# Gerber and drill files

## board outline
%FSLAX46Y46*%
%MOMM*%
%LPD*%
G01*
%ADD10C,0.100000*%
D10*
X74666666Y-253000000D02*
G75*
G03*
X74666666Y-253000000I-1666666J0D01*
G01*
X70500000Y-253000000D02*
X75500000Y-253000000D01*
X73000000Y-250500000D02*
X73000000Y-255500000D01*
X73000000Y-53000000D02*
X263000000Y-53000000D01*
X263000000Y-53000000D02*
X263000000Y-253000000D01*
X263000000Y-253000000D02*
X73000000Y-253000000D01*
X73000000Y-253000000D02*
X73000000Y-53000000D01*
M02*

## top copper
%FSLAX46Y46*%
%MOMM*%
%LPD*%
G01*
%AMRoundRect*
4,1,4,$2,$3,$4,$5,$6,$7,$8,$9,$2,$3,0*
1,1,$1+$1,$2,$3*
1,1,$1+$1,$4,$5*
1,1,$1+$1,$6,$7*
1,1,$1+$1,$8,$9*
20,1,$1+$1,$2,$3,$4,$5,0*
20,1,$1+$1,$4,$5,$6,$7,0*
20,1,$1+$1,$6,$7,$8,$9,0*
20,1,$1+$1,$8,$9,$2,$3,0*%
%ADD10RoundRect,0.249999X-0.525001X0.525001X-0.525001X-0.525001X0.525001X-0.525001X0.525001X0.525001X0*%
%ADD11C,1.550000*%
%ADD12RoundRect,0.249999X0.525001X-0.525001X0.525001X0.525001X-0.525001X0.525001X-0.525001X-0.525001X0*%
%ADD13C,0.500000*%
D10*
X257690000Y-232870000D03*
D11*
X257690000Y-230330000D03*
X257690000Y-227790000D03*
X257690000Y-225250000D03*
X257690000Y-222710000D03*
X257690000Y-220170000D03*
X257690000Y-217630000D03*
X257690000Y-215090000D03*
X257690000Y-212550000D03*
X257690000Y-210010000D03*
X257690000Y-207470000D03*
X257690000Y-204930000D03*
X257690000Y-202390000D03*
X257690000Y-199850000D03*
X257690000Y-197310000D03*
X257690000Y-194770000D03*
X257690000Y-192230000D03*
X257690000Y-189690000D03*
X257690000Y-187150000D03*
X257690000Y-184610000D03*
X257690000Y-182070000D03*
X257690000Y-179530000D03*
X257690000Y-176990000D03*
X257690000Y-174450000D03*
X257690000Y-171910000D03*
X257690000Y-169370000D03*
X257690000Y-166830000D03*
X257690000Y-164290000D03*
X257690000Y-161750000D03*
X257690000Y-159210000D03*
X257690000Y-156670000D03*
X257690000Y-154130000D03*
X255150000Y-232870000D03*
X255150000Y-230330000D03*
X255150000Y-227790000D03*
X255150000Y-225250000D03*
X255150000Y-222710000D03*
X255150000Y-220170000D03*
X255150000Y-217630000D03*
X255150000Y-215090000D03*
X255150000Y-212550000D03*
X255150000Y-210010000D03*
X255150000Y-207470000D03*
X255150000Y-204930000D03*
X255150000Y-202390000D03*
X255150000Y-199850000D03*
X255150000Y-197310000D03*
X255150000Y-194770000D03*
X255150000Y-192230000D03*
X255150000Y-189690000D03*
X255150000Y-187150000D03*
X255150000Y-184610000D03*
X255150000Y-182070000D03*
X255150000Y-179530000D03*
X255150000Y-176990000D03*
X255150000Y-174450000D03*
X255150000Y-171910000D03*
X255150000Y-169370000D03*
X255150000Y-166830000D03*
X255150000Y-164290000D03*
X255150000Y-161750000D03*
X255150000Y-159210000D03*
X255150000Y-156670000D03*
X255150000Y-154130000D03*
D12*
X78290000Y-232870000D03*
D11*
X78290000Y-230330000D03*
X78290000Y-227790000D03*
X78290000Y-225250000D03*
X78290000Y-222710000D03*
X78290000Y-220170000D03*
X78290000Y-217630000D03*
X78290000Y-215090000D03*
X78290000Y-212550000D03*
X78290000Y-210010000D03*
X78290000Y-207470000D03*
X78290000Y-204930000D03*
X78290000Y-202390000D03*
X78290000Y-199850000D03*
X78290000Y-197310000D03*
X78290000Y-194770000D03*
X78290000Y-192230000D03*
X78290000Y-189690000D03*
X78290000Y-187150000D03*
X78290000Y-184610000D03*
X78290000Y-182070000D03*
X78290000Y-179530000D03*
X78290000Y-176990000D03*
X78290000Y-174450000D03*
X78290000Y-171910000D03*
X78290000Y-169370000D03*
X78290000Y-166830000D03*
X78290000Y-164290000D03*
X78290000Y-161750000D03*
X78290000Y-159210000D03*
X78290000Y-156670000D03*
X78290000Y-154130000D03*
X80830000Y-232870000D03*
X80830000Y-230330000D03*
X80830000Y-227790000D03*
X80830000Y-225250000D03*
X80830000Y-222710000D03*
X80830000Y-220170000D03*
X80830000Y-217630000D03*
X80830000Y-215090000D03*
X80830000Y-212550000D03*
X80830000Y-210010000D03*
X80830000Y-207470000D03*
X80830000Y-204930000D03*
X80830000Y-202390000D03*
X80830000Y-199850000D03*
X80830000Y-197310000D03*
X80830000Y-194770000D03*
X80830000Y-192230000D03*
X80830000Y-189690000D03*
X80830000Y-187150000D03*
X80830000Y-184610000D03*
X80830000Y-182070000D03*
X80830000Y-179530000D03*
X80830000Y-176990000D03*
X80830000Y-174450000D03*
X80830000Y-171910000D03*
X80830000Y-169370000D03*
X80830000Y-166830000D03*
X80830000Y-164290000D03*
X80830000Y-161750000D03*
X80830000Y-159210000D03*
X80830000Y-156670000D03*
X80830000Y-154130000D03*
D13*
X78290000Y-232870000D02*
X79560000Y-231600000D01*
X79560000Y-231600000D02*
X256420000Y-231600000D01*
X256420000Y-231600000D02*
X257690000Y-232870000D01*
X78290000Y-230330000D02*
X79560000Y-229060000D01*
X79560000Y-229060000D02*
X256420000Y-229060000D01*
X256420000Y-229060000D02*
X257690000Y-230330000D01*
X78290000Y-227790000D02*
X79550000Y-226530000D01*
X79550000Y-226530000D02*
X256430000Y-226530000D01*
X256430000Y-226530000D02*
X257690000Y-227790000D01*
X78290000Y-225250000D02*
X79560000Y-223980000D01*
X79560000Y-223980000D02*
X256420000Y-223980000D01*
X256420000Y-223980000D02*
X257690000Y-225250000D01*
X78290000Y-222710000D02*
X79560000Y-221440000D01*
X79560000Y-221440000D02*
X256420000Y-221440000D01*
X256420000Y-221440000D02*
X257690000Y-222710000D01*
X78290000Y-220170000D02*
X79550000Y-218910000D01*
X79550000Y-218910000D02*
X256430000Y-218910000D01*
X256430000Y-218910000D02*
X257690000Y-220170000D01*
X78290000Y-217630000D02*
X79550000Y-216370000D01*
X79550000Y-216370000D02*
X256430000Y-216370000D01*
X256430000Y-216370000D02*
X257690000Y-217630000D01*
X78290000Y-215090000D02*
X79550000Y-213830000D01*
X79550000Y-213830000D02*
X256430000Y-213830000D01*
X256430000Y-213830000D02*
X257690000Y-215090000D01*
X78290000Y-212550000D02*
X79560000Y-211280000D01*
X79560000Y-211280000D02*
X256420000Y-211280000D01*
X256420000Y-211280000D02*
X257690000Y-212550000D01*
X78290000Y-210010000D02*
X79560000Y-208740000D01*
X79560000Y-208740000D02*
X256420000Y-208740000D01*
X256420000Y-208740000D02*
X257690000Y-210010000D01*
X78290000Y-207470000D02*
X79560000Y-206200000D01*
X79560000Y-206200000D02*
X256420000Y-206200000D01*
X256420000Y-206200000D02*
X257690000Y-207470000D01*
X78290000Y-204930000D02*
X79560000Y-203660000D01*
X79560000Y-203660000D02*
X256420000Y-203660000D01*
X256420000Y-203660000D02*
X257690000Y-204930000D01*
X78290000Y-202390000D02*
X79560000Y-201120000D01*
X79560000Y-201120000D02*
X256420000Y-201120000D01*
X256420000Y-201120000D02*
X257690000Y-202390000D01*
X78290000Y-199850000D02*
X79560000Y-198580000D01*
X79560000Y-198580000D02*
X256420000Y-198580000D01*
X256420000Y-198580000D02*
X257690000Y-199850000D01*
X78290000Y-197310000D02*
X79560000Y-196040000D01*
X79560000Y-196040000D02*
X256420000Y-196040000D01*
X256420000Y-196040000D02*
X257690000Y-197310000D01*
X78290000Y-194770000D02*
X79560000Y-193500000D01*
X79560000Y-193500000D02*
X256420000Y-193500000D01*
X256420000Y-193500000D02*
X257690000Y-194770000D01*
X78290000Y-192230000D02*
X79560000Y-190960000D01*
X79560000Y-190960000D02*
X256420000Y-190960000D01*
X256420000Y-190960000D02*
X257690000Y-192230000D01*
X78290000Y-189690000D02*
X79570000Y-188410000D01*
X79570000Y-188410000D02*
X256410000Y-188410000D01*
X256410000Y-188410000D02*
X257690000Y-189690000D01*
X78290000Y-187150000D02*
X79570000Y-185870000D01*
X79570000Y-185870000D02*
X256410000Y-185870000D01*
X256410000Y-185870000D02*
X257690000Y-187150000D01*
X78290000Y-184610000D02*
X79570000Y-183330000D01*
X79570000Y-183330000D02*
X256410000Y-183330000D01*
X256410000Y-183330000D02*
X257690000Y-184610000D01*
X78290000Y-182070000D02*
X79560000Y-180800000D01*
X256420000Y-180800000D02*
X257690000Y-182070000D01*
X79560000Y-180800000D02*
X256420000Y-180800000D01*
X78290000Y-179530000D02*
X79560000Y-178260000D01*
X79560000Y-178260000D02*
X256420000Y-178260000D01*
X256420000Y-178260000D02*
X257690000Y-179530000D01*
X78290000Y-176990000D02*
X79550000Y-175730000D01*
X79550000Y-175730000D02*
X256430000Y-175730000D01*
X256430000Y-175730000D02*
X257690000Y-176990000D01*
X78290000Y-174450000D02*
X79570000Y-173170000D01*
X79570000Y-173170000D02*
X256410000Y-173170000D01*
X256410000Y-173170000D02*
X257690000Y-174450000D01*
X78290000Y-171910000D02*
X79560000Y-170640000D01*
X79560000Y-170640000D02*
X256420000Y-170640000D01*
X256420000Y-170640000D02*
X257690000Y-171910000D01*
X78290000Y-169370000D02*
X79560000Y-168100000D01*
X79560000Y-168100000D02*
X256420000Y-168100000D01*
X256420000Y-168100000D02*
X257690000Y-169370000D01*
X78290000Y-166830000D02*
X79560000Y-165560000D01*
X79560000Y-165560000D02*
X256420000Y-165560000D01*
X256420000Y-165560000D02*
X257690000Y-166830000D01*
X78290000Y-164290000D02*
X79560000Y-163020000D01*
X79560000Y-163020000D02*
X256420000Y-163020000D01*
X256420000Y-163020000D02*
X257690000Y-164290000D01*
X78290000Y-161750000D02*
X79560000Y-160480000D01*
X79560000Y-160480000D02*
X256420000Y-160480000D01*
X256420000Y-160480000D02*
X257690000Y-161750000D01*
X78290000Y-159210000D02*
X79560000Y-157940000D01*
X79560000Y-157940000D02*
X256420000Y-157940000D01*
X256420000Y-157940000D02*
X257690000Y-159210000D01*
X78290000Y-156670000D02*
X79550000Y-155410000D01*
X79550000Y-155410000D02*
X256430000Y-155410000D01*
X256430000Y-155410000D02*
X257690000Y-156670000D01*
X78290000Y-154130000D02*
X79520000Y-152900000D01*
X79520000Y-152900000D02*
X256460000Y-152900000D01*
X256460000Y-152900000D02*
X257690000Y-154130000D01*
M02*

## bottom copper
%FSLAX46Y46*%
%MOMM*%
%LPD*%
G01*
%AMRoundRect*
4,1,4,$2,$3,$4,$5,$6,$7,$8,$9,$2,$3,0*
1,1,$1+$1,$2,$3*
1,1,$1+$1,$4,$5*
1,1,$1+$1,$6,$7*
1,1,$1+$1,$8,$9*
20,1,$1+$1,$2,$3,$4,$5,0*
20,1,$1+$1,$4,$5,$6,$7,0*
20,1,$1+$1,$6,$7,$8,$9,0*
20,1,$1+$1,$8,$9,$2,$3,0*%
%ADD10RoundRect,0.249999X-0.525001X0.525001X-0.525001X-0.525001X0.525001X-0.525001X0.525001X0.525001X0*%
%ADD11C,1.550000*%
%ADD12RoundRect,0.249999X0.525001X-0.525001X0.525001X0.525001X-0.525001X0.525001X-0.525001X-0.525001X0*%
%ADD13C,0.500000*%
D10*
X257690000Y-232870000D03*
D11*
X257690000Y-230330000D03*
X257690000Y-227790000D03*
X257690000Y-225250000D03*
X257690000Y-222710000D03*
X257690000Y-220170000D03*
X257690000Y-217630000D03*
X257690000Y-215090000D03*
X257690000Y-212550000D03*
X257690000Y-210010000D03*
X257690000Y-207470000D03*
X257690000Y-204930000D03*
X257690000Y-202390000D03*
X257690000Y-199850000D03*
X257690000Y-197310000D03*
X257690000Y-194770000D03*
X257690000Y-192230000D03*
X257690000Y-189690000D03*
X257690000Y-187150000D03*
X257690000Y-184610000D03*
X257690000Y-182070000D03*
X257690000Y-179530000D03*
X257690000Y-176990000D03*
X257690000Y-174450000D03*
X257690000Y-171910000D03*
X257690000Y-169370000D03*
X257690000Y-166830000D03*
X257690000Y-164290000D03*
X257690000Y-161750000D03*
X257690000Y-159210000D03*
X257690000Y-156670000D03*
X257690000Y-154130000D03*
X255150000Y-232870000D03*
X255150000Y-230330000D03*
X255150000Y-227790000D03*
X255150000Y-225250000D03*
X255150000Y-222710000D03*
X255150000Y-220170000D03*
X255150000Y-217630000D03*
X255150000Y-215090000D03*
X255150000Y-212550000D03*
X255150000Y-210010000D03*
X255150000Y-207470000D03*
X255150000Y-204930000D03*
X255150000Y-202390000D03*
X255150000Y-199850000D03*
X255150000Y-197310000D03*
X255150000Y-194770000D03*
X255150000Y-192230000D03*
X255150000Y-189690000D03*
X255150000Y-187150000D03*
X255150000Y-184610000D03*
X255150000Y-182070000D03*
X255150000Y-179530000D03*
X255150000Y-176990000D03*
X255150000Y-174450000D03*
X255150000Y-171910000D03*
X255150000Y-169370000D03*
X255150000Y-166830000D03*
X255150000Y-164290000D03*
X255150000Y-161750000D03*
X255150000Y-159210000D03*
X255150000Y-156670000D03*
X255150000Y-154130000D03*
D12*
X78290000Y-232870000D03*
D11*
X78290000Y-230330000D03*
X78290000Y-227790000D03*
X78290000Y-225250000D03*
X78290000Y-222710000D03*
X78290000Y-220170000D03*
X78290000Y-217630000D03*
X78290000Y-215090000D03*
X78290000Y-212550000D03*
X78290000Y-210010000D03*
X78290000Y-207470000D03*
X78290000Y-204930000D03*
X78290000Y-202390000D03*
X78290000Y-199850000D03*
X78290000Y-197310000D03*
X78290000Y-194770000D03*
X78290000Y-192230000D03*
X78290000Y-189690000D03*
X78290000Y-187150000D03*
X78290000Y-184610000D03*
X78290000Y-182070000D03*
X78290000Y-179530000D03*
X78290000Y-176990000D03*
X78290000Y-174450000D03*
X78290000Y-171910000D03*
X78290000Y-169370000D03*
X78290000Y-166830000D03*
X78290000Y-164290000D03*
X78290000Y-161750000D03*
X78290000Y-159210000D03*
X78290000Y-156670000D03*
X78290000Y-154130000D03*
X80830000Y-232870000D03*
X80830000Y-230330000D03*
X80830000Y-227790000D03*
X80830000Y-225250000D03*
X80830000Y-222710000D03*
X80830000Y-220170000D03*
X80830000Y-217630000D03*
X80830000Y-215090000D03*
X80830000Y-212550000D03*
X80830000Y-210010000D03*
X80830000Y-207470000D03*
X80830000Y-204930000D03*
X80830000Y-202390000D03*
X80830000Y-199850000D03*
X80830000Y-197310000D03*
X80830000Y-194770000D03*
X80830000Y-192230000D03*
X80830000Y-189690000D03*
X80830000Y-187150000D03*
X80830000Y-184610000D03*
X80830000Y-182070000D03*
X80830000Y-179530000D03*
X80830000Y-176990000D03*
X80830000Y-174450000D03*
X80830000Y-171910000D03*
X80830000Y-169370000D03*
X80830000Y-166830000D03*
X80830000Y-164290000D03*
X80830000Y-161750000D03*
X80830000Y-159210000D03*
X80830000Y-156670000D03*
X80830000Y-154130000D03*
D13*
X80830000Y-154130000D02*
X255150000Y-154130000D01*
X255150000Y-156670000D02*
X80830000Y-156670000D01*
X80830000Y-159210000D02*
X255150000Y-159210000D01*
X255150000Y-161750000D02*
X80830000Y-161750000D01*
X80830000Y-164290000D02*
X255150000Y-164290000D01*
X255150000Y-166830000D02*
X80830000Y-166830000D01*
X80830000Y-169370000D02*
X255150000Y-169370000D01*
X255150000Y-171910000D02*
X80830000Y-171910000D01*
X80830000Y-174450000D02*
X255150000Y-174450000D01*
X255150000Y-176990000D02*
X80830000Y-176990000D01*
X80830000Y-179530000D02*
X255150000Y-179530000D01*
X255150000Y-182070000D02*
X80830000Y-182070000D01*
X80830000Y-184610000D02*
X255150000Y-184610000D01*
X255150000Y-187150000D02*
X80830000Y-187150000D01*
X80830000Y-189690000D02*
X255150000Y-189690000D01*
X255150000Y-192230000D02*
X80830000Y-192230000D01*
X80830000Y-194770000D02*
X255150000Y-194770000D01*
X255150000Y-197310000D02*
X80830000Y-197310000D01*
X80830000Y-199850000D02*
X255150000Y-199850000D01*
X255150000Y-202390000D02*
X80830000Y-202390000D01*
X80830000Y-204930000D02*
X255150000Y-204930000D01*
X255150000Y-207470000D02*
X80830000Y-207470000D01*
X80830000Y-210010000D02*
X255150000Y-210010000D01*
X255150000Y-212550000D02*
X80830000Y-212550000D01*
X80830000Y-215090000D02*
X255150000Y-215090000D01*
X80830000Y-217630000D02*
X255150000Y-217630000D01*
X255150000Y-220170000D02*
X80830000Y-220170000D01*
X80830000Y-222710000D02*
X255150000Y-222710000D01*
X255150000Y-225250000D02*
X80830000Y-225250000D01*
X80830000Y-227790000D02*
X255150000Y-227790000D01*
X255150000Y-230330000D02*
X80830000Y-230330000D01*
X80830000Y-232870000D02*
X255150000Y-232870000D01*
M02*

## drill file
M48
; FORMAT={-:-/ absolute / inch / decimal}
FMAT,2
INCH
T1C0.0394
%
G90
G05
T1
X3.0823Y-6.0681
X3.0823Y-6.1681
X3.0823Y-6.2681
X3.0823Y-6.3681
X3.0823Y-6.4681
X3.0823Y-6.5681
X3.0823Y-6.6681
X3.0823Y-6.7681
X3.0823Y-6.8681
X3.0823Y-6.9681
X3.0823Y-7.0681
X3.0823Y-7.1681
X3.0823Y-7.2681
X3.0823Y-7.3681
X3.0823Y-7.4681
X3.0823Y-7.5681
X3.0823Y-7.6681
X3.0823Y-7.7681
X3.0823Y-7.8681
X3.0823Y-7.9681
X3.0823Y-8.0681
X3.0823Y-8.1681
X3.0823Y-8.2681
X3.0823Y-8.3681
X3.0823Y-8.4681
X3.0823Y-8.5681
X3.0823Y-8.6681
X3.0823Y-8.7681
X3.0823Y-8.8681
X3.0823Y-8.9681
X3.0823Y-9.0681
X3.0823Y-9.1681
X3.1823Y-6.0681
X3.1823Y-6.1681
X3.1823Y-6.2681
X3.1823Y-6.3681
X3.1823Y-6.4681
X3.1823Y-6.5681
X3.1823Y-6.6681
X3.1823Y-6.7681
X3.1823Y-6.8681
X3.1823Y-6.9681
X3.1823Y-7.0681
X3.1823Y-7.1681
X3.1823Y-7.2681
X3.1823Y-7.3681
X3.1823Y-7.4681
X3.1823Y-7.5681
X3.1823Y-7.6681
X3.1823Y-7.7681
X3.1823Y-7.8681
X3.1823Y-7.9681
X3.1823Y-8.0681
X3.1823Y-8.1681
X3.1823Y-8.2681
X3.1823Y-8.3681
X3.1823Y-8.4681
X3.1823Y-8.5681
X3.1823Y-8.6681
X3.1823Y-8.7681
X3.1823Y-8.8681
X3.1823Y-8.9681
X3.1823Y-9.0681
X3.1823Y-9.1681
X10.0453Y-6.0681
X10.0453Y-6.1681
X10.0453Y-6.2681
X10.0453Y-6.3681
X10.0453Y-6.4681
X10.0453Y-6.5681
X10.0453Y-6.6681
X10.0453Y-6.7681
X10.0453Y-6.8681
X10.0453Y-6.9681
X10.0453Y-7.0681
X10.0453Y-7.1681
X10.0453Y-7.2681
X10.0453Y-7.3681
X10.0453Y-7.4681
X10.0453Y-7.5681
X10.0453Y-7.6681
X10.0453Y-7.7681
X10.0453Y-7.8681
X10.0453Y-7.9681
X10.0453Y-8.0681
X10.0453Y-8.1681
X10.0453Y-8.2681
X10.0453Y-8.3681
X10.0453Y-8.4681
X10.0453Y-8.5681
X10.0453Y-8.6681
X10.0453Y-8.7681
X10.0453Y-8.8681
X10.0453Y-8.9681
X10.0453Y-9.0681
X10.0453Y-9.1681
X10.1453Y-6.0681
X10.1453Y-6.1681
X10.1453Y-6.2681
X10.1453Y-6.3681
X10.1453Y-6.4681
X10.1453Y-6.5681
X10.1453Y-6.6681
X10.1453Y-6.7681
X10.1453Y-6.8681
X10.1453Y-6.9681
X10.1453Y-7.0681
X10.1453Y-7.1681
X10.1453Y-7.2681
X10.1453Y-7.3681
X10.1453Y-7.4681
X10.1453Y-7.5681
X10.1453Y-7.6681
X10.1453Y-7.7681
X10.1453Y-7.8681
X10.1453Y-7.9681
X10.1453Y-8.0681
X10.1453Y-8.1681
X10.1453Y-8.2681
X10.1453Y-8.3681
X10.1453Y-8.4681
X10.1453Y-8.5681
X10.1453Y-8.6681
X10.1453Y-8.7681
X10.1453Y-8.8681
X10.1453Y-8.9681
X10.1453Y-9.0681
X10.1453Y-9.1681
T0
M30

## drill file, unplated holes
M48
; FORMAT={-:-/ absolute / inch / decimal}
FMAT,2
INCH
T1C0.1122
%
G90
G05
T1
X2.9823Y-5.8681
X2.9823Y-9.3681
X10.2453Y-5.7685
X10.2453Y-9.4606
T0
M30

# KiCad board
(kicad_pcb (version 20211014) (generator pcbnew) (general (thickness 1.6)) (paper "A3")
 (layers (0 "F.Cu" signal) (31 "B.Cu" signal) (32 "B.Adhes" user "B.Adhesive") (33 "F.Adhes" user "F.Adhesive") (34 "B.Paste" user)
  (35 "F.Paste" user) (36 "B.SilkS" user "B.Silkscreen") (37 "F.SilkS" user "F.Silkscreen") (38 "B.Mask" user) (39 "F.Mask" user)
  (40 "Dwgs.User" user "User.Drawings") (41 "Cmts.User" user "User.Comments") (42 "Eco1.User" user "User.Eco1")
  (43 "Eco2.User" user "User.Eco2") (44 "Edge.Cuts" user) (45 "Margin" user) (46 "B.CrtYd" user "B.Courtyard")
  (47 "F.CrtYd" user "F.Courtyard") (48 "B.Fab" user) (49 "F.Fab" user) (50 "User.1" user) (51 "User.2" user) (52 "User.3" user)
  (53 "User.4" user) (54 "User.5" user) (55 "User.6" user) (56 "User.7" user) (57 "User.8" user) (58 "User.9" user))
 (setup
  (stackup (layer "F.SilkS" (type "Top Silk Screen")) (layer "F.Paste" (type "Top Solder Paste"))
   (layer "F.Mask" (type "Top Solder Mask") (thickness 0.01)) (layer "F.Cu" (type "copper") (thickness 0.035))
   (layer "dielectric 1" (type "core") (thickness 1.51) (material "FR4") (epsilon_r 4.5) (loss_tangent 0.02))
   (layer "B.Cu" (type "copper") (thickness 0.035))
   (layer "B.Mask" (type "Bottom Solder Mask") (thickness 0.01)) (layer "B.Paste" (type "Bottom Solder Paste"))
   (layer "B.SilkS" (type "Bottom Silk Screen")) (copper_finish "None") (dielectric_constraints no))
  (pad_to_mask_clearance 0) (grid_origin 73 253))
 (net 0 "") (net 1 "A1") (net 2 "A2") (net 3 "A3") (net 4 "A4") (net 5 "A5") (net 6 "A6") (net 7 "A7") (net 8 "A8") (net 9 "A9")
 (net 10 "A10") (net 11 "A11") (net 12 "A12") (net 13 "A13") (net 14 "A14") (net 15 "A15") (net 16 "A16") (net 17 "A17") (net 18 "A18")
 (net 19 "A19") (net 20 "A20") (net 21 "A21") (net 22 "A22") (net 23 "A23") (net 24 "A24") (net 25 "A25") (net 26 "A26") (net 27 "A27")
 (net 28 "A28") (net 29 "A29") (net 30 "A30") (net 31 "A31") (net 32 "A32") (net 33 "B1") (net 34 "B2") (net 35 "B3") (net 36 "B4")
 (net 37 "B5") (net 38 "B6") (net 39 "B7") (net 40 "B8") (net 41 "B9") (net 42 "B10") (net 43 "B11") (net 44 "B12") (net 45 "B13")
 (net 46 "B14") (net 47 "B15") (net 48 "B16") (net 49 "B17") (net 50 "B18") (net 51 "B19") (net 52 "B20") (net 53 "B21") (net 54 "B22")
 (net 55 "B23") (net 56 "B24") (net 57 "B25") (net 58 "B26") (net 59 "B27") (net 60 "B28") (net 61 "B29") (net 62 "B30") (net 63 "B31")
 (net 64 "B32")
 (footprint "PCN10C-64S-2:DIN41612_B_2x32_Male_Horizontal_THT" (layer "F.Cu") (at 257.69 232.87 -90)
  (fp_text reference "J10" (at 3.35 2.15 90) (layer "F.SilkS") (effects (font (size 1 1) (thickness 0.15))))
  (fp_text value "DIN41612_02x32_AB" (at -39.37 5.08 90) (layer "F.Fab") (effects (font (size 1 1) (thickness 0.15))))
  (pad "" np_thru_hole circle (at -86.35 -2.54 270) (size 2.85 2.85) (drill 2.85) (layers F&B.Cu *.Mask))
  (pad "" np_thru_hole circle (at 7.43 -2.54 270) (size 2.85 2.85) (drill 2.85) (layers F&B.Cu *.Mask))
  (pad "a1" thru_hole roundrect (at 0 0 270) (size 1.55 1.55) (drill 1) (layers *.Cu *.Mask) (roundrect_rratio 0.1612896774) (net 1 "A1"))
  (pad "a2" thru_hole circle (at -2.54 0 270) (size 1.55 1.55) (drill 1) (layers *.Cu *.Mask) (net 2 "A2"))
  (pad "a3" thru_hole circle (at -5.08 0 270) (size 1.55 1.55) (drill 1) (layers *.Cu *.Mask) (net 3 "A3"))
  (pad "a4" thru_hole circle (at -7.62 0 270) (size 1.55 1.55) (drill 1) (layers *.Cu *.Mask) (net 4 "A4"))
  (pad "a5" thru_hole circle (at -10.16 0 270) (size 1.55 1.55) (drill 1) (layers *.Cu *.Mask) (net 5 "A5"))
  (pad "a6" thru_hole circle (at -12.7 0 270) (size 1.55 1.55) (drill 1) (layers *.Cu *.Mask) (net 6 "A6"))
  (pad "a7" thru_hole circle (at -15.24 0 270) (size 1.55 1.55) (drill 1) (layers *.Cu *.Mask) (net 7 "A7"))
  (pad "a8" thru_hole circle (at -17.78 0 270) (size 1.55 1.55) (drill 1) (layers *.Cu *.Mask) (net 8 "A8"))
  (pad "a9" thru_hole circle (at -20.32 0 270) (size 1.55 1.55) (drill 1) (layers *.Cu *.Mask) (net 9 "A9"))
  (pad "a10" thru_hole circle (at -22.86 0 270) (size 1.55 1.55) (drill 1) (layers *.Cu *.Mask) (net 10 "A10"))
  (pad "a11" thru_hole circle (at -25.4 0 270) (size 1.55 1.55) (drill 1) (layers *.Cu *.Mask) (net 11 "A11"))
  (pad "a12" thru_hole circle (at -27.94 0 270) (size 1.55 1.55) (drill 1) (layers *.Cu *.Mask) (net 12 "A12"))
  (pad "a13" thru_hole circle (at -30.48 0 270) (size 1.55 1.55) (drill 1) (layers *.Cu *.Mask) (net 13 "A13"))
  (pad "a14" thru_hole circle (at -33.02 0 270) (size 1.55 1.55) (drill 1) (layers *.Cu *.Mask) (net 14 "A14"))
  (pad "a15" thru_hole circle (at -35.56 0 270) (size 1.55 1.55) (drill 1) (layers *.Cu *.Mask) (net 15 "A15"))
  (pad "a16" thru_hole circle (at -38.1 0 270) (size 1.55 1.55) (drill 1) (layers *.Cu *.Mask) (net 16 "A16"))
  (pad "a17" thru_hole circle (at -40.64 0 270) (size 1.55 1.55) (drill 1) (layers *.Cu *.Mask) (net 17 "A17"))
  (pad "a18" thru_hole circle (at -43.18 0 270) (size 1.55 1.55) (drill 1) (layers *.Cu *.Mask) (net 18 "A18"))
  (pad "a19" thru_hole circle (at -45.72 0 270) (size 1.55 1.55) (drill 1) (layers *.Cu *.Mask) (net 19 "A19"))
  (pad "a20" thru_hole circle (at -48.26 0 270) (size 1.55 1.55) (drill 1) (layers *.Cu *.Mask) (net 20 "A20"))
  (pad "a21" thru_hole circle (at -50.8 0 270) (size 1.55 1.55) (drill 1) (layers *.Cu *.Mask) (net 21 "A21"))
  (pad "a22" thru_hole circle (at -53.34 0 270) (size 1.55 1.55) (drill 1) (layers *.Cu *.Mask) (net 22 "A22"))
  (pad "a23" thru_hole circle (at -55.88 0 270) (size 1.55 1.55) (drill 1) (layers *.Cu *.Mask) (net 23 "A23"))
  (pad "a24" thru_hole circle (at -58.42 0 270) (size 1.55 1.55) (drill 1) (layers *.Cu *.Mask) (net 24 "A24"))
  (pad "a25" thru_hole circle (at -60.96 0 270) (size 1.55 1.55) (drill 1) (layers *.Cu *.Mask) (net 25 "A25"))
  (pad "a26" thru_hole circle (at -63.5 0 270) (size 1.55 1.55) (drill 1) (layers *.Cu *.Mask) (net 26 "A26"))
  (pad "a27" thru_hole circle (at -66.04 0 270) (size 1.55 1.55) (drill 1) (layers *.Cu *.Mask) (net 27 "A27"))
  (pad "a28" thru_hole circle (at -68.58 0 270) (size 1.55 1.55) (drill 1) (layers *.Cu *.Mask) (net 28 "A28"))
  (pad "a29" thru_hole circle (at -71.12 0 270) (size 1.55 1.55) (drill 1) (layers *.Cu *.Mask) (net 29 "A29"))
  (pad "a30" thru_hole circle (at -73.66 0 270) (size 1.55 1.55) (drill 1) (layers *.Cu *.Mask) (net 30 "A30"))
  (pad "a31" thru_hole circle (at -76.2 0 270) (size 1.55 1.55) (drill 1) (layers *.Cu *.Mask) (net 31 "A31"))
  (pad "a32" thru_hole circle (at -78.74 0 270) (size 1.55 1.55) (drill 1) (layers *.Cu *.Mask) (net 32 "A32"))
  (pad "b1" thru_hole circle (at 0 2.54 270) (size 1.55 1.55) (drill 1) (layers *.Cu *.Mask) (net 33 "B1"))
  (pad "b2" thru_hole circle (at -2.54 2.54 270) (size 1.55 1.55) (drill 1) (layers *.Cu *.Mask) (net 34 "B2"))
  (pad "b3" thru_hole circle (at -5.08 2.54 270) (size 1.55 1.55) (drill 1) (layers *.Cu *.Mask) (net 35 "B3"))
  (pad "b4" thru_hole circle (at -7.62 2.54 270) (size 1.55 1.55) (drill 1) (layers *.Cu *.Mask) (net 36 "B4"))
  (pad "b5" thru_hole circle (at -10.16 2.54 270) (size 1.55 1.55) (drill 1) (layers *.Cu *.Mask) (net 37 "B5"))
  (pad "b6" thru_hole circle (at -12.7 2.54 270) (size 1.55 1.55) (drill 1) (layers *.Cu *.Mask) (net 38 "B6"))
  (pad "b7" thru_hole circle (at -15.24 2.54 270) (size 1.55 1.55) (drill 1) (layers *.Cu *.Mask) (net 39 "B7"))
  (pad "b8" thru_hole circle (at -17.78 2.54 270) (size 1.55 1.55) (drill 1) (layers *.Cu *.Mask) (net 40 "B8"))
  (pad "b9" thru_hole circle (at -20.32 2.54 270) (size 1.55 1.55) (drill 1) (layers *.Cu *.Mask) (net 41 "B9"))
  (pad "b10" thru_hole circle (at -22.86 2.54 270) (size 1.55 1.55) (drill 1) (layers *.Cu *.Mask) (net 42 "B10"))
  (pad "b11" thru_hole circle (at -25.4 2.54 270) (size 1.55 1.55) (drill 1) (layers *.Cu *.Mask) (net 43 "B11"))
  (pad "b12" thru_hole circle (at -27.94 2.54 270) (size 1.55 1.55) (drill 1) (layers *.Cu *.Mask) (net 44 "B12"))
  (pad "b13" thru_hole circle (at -30.48 2.54 270) (size 1.55 1.55) (drill 1) (layers *.Cu *.Mask) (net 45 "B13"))
  (pad "b14" thru_hole circle (at -33.02 2.54 270) (size 1.55 1.55) (drill 1) (layers *.Cu *.Mask) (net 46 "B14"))
  (pad "b15" thru_hole circle (at -35.56 2.54 270) (size 1.55 1.55) (drill 1) (layers *.Cu *.Mask) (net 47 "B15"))
  (pad "b16" thru_hole circle (at -38.1 2.54 270) (size 1.55 1.55) (drill 1) (layers *.Cu *.Mask) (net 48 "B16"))
  (pad "b17" thru_hole circle (at -40.64 2.54 270) (size 1.55 1.55) (drill 1) (layers *.Cu *.Mask) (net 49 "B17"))
  (pad "b18" thru_hole circle (at -43.18 2.54 270) (size 1.55 1.55) (drill 1) (layers *.Cu *.Mask) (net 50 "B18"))
  (pad "b19" thru_hole circle (at -45.72 2.54 270) (size 1.55 1.55) (drill 1) (layers *.Cu *.Mask) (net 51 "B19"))
  (pad "b20" thru_hole circle (at -48.26 2.54 270) (size 1.55 1.55) (drill 1) (layers *.Cu *.Mask) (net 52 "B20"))
  (pad "b21" thru_hole circle (at -50.8 2.54 270) (size 1.55 1.55) (drill 1) (layers *.Cu *.Mask) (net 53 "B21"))
  (pad "b22" thru_hole circle (at -53.34 2.54 270) (size 1.55 1.55) (drill 1) (layers *.Cu *.Mask) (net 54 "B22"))
  (pad "b23" thru_hole circle (at -55.88 2.54 270) (size 1.55 1.55) (drill 1) (layers *.Cu *.Mask) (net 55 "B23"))
  (pad "b24" thru_hole circle (at -58.42 2.54 270) (size 1.55 1.55) (drill 1) (layers *.Cu *.Mask) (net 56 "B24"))
  (pad "b25" thru_hole circle (at -60.96 2.54 270) (size 1.55 1.55) (drill 1) (layers *.Cu *.Mask) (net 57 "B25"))
  (pad "b26" thru_hole circle (at -63.5 2.54 270) (size 1.55 1.55) (drill 1) (layers *.Cu *.Mask) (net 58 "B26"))
  (pad "b27" thru_hole circle (at -66.04 2.54 270) (size 1.55 1.55) (drill 1) (layers *.Cu *.Mask) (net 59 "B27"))
  (pad "b28" thru_hole circle (at -68.58 2.54 270) (size 1.55 1.55) (drill 1) (layers *.Cu *.Mask) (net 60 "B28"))
  (pad "b29" thru_hole circle (at -71.12 2.54 270) (size 1.55 1.55) (drill 1) (layers *.Cu *.Mask) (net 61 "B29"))
  (pad "b30" thru_hole circle (at -73.66 2.54 270) (size 1.55 1.55) (drill 1) (layers *.Cu *.Mask) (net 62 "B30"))
  (pad "b31" thru_hole circle (at -76.2 2.54 270) (size 1.55 1.55) (drill 1) (layers *.Cu *.Mask) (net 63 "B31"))
  (pad "b32" thru_hole circle (at -78.74 2.54 270) (size 1.55 1.55) (drill 1) (layers *.Cu *.Mask) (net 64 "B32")))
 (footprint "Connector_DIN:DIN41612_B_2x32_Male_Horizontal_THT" (layer "F.Cu") (at 78.29 232.87 90)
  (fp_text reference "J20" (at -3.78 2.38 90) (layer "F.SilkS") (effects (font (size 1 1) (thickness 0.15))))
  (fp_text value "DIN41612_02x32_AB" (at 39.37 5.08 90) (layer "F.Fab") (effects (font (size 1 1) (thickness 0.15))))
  (pad "" np_thru_hole circle (at -5.08 -2.54 90) (size 2.85 2.85) (drill 2.85) (layers *.Cu *.Mask))
  (pad "" np_thru_hole circle (at 83.82 -2.54 90) (size 2.85 2.85) (drill 2.85) (layers *.Cu *.Mask))
  (pad "a1" thru_hole roundrect (at 0 0 90) (size 1.55 1.55) (drill 1) (layers *.Cu *.Mask) (roundrect_rratio 0.1612896774) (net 1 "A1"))
  (pad "a2" thru_hole circle (at 2.54 0 90) (size 1.55 1.55) (drill 1) (layers *.Cu *.Mask) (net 2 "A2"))
  (pad "a3" thru_hole circle (at 5.08 0 90) (size 1.55 1.55) (drill 1) (layers *.Cu *.Mask) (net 3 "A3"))
  (pad "a4" thru_hole circle (at 7.62 0 90) (size 1.55 1.55) (drill 1) (layers *.Cu *.Mask) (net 4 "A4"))
  (pad "a5" thru_hole circle (at 10.16 0 90) (size 1.55 1.55) (drill 1) (layers *.Cu *.Mask) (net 5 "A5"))
  (pad "a6" thru_hole circle (at 12.7 0 90) (size 1.55 1.55) (drill 1) (layers *.Cu *.Mask) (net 6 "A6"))
  (pad "a7" thru_hole circle (at 15.24 0 90) (size 1.55 1.55) (drill 1) (layers *.Cu *.Mask) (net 7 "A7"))
  (pad "a8" thru_hole circle (at 17.78 0 90) (size 1.55 1.55) (drill 1) (layers *.Cu *.Mask) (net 8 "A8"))
  (pad "a9" thru_hole circle (at 20.32 0 90) (size 1.55 1.55) (drill 1) (layers *.Cu *.Mask) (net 9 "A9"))
  (pad "a10" thru_hole circle (at 22.86 0 90) (size 1.55 1.55) (drill 1) (layers *.Cu *.Mask) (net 10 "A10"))
  (pad "a11" thru_hole circle (at 25.4 0 90) (size 1.55 1.55) (drill 1) (layers *.Cu *.Mask) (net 11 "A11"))
  (pad "a12" thru_hole circle (at 27.94 0 90) (size 1.55 1.55) (drill 1) (layers *.Cu *.Mask) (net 12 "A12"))
  (pad "a13" thru_hole circle (at 30.48 0 90) (size 1.55 1.55) (drill 1) (layers *.Cu *.Mask) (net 13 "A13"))
  (pad "a14" thru_hole circle (at 33.02 0 90) (size 1.55 1.55) (drill 1) (layers *.Cu *.Mask) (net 14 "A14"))
  (pad "a15" thru_hole circle (at 35.56 0 90) (size 1.55 1.55) (drill 1) (layers *.Cu *.Mask) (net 15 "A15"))
  (pad "a16" thru_hole circle (at 38.1 0 90) (size 1.55 1.55) (drill 1) (layers *.Cu *.Mask) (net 16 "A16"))
  (pad "a17" thru_hole circle (at 40.64 0 90) (size 1.55 1.55) (drill 1) (layers *.Cu *.Mask) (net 17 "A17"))
  (pad "a18" thru_hole circle (at 43.18 0 90) (size 1.55 1.55) (drill 1) (layers *.Cu *.Mask) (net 18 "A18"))
  (pad "a19" thru_hole circle (at 45.72 0 90) (size 1.55 1.55) (drill 1) (layers *.Cu *.Mask) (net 19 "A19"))
  (pad "a20" thru_hole circle (at 48.26 0 90) (size 1.55 1.55) (drill 1) (layers *.Cu *.Mask) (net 20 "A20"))
  (pad "a21" thru_hole circle (at 50.8 0 90) (size 1.55 1.55) (drill 1) (layers *.Cu *.Mask) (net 21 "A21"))
  (pad "a22" thru_hole circle (at 53.34 0 90) (size 1.55 1.55) (drill 1) (layers *.Cu *.Mask) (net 22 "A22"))
  (pad "a23" thru_hole circle (at 55.88 0 90) (size 1.55 1.55) (drill 1) (layers *.Cu *.Mask) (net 23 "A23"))
  (pad "a24" thru_hole circle (at 58.42 0 90) (size 1.55 1.55) (drill 1) (layers *.Cu *.Mask) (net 24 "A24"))
  (pad "a25" thru_hole circle (at 60.96 0 90) (size 1.55 1.55) (drill 1) (layers *.Cu *.Mask) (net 25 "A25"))
  (pad "a26" thru_hole circle (at 63.5 0 90) (size 1.55 1.55) (drill 1) (layers *.Cu *.Mask) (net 26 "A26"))
  (pad "a27" thru_hole circle (at 66.04 0 90) (size 1.55 1.55) (drill 1) (layers *.Cu *.Mask) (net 27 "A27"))
  (pad "a28" thru_hole circle (at 68.58 0 90) (size 1.55 1.55) (drill 1) (layers *.Cu *.Mask) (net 28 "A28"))
  (pad "a29" thru_hole circle (at 71.12 0 90) (size 1.55 1.55) (drill 1) (layers *.Cu *.Mask) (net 29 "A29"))
  (pad "a30" thru_hole circle (at 73.66 0 90) (size 1.55 1.55) (drill 1) (layers *.Cu *.Mask) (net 30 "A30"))
  (pad "a31" thru_hole circle (at 76.2 0 90) (size 1.55 1.55) (drill 1) (layers *.Cu *.Mask) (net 31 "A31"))
  (pad "a32" thru_hole circle (at 78.74 0 90) (size 1.55 1.55) (drill 1) (layers *.Cu *.Mask) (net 32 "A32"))
  (pad "b1" thru_hole circle (at 0 2.54 90) (size 1.55 1.55) (drill 1) (layers *.Cu *.Mask) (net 33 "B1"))
  (pad "b2" thru_hole circle (at 2.54 2.54 90) (size 1.55 1.55) (drill 1) (layers *.Cu *.Mask) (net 34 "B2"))
  (pad "b3" thru_hole circle (at 5.08 2.54 90) (size 1.55 1.55) (drill 1) (layers *.Cu *.Mask) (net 35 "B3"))
  (pad "b4" thru_hole circle (at 7.62 2.54 90) (size 1.55 1.55) (drill 1) (layers *.Cu *.Mask) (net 36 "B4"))
  (pad "b5" thru_hole circle (at 10.16 2.54 90) (size 1.55 1.55) (drill 1) (layers *.Cu *.Mask) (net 37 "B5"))
  (pad "b6" thru_hole circle (at 12.7 2.54 90) (size 1.55 1.55) (drill 1) (layers *.Cu *.Mask) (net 38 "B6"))
  (pad "b7" thru_hole circle (at 15.24 2.54 90) (size 1.55 1.55) (drill 1) (layers *.Cu *.Mask) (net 39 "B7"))
  (pad "b8" thru_hole circle (at 17.78 2.54 90) (size 1.55 1.55) (drill 1) (layers *.Cu *.Mask) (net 40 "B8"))
  (pad "b9" thru_hole circle (at 20.32 2.54 90) (size 1.55 1.55) (drill 1) (layers *.Cu *.Mask) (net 41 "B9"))
  (pad "b10" thru_hole circle (at 22.86 2.54 90) (size 1.55 1.55) (drill 1) (layers *.Cu *.Mask) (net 42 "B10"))
  (pad "b11" thru_hole circle (at 25.4 2.54 90) (size 1.55 1.55) (drill 1) (layers *.Cu *.Mask) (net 43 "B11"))
  (pad "b12" thru_hole circle (at 27.94 2.54 90) (size 1.55 1.55) (drill 1) (layers *.Cu *.Mask) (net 44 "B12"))
  (pad "b13" thru_hole circle (at 30.48 2.54 90) (size 1.55 1.55) (drill 1) (layers *.Cu *.Mask) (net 45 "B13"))
  (pad "b14" thru_hole circle (at 33.02 2.54 90) (size 1.55 1.55) (drill 1) (layers *.Cu *.Mask) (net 46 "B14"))
  (pad "b15" thru_hole circle (at 35.56 2.54 90) (size 1.55 1.55) (drill 1) (layers *.Cu *.Mask) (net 47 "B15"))
  (pad "b16" thru_hole circle (at 38.1 2.54 90) (size 1.55 1.55) (drill 1) (layers *.Cu *.Mask) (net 48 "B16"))
  (pad "b17" thru_hole circle (at 40.64 2.54 90) (size 1.55 1.55) (drill 1) (layers *.Cu *.Mask) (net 49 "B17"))
  (pad "b18" thru_hole circle (at 43.18 2.54 90) (size 1.55 1.55) (drill 1) (layers *.Cu *.Mask) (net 50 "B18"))
  (pad "b19" thru_hole circle (at 45.72 2.54 90) (size 1.55 1.55) (drill 1) (layers *.Cu *.Mask) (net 51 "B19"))
  (pad "b20" thru_hole circle (at 48.26 2.54 90) (size 1.55 1.55) (drill 1) (layers *.Cu *.Mask) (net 52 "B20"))
  (pad "b21" thru_hole circle (at 50.8 2.54 90) (size 1.55 1.55) (drill 1) (layers *.Cu *.Mask) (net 53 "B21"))
  (pad "b22" thru_hole circle (at 53.34 2.54 90) (size 1.55 1.55) (drill 1) (layers *.Cu *.Mask) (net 54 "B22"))
  (pad "b23" thru_hole circle (at 55.88 2.54 90) (size 1.55 1.55) (drill 1) (layers *.Cu *.Mask) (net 55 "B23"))
  (pad "b24" thru_hole circle (at 58.42 2.54 90) (size 1.55 1.55) (drill 1) (layers *.Cu *.Mask) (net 56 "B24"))
  (pad "b25" thru_hole circle (at 60.96 2.54 90) (size 1.55 1.55) (drill 1) (layers *.Cu *.Mask) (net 57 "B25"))
  (pad "b26" thru_hole circle (at 63.5 2.54 90) (size 1.55 1.55) (drill 1) (layers *.Cu *.Mask) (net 58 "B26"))
  (pad "b27" thru_hole circle (at 66.04 2.54 90) (size 1.55 1.55) (drill 1) (layers *.Cu *.Mask) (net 59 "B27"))
  (pad "b28" thru_hole circle (at 68.58 2.54 90) (size 1.55 1.55) (drill 1) (layers *.Cu *.Mask) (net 60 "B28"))
  (pad "b29" thru_hole circle (at 71.12 2.54 90) (size 1.55 1.55) (drill 1) (layers *.Cu *.Mask) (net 61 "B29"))
  (pad "b30" thru_hole circle (at 73.66 2.54 90) (size 1.55 1.55) (drill 1) (layers *.Cu *.Mask) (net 62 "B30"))
  (pad "b31" thru_hole circle (at 76.2 2.54 90) (size 1.55 1.55) (drill 1) (layers *.Cu *.Mask) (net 63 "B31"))
  (pad "b32" thru_hole circle (at 78.74 2.54 90) (size 1.55 1.55) (drill 1) (layers *.Cu *.Mask) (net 64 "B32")))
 (gr_rect (start 73 53) (end 263 253) (layer "Edge.Cuts") (width 0.1) (fill none))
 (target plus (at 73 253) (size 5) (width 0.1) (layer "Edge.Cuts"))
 (segment (start 78.29 232.87) (end 79.56 231.6) (width 0.5) (layer "F.Cu") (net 1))
 (segment (start 256.42 231.6) (end 257.69 232.87) (width 0.5) (layer "F.Cu") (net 1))
 (segment (start 79.56 231.6) (end 256.42 231.6) (width 0.5) (layer "F.Cu") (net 1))
 (segment (start 256.42 229.06) (end 257.69 230.33) (width 0.5) (layer "F.Cu") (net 2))
 (segment (start 79.56 229.06) (end 256.42 229.06) (width 0.5) (layer "F.Cu") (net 2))
 (segment (start 78.29 230.33) (end 79.56 229.06) (width 0.5) (layer "F.Cu") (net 2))
 (segment (start 256.43 226.53) (end 257.69 227.79) (width 0.5) (layer "F.Cu") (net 3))
 (segment (start 78.29 227.79) (end 79.55 226.53) (width 0.5) (layer "F.Cu") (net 3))
 (segment (start 79.55 226.53) (end 256.43 226.53) (width 0.5) (layer "F.Cu") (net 3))
 (segment (start 78.29 225.25) (end 79.56 223.98) (width 0.5) (layer "F.Cu") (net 4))
 (segment (start 256.42 223.98) (end 257.69 225.25) (width 0.5) (layer "F.Cu") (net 4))
 (segment (start 79.56 223.98) (end 256.42 223.98) (width 0.5) (layer "F.Cu") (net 4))
 (segment (start 79.56 221.44) (end 256.42 221.44) (width 0.5) (layer "F.Cu") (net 5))
 (segment (start 78.29 222.71) (end 79.56 221.44) (width 0.5) (layer "F.Cu") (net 5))
 (segment (start 256.42 221.44) (end 257.69 222.71) (width 0.5) (layer "F.Cu") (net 5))
 (segment (start 256.43 218.91) (end 257.69 220.17) (width 0.5) (layer "F.Cu") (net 6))
 (segment (start 78.29 220.17) (end 79.55 218.91) (width 0.5) (layer "F.Cu") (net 6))
 (segment (start 79.55 218.91) (end 256.43 218.91) (width 0.5) (layer "F.Cu") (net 6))
 (segment (start 78.29 217.63) (end 79.55 216.37) (width 0.5) (layer "F.Cu") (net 7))
 (segment (start 79.55 216.37) (end 256.43 216.37) (width 0.5) (layer "F.Cu") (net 7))
 (segment (start 256.43 216.37) (end 257.69 217.63) (width 0.5) (layer "F.Cu") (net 7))
 (segment (start 78.29 215.09) (end 79.55 213.83) (width 0.5) (layer "F.Cu") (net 8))
 (segment (start 79.55 213.83) (end 256.43 213.83) (width 0.5) (layer "F.Cu") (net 8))
 (segment (start 256.43 213.83) (end 257.69 215.09) (width 0.5) (layer "F.Cu") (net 8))
 (segment (start 79.56 211.28) (end 256.42 211.28) (width 0.5) (layer "F.Cu") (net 9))
 (segment (start 78.29 212.55) (end 79.56 211.28) (width 0.5) (layer "F.Cu") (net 9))
 (segment (start 256.42 211.28) (end 257.69 212.55) (width 0.5) (layer "F.Cu") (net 9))
 (segment (start 79.56 208.74) (end 256.42 208.74) (width 0.5) (layer "F.Cu") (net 10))
 (segment (start 78.29 210.01) (end 79.56 208.74) (width 0.5) (layer "F.Cu") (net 10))
 (segment (start 256.42 208.74) (end 257.69 210.01) (width 0.5) (layer "F.Cu") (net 10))
 (segment (start 79.56 206.2) (end 256.42 206.2) (width 0.5) (layer "F.Cu") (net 11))
 (segment (start 256.42 206.2) (end 257.69 207.47) (width 0.5) (layer "F.Cu") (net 11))
 (segment (start 78.29 207.47) (end 79.56 206.2) (width 0.5) (layer "F.Cu") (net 11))
 (segment (start 78.29 204.93) (end 79.56 203.66) (width 0.5) (layer "F.Cu") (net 12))
 (segment (start 79.56 203.66) (end 256.42 203.66) (width 0.5) (layer "F.Cu") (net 12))
 (segment (start 256.42 203.66) (end 257.69 204.93) (width 0.5) (layer "F.Cu") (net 12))
 (segment (start 79.56 201.12) (end 256.42 201.12) (width 0.5) (layer "F.Cu") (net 13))
 (segment (start 256.42 201.12) (end 257.69 202.39) (width 0.5) (layer "F.Cu") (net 13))
 (segment (start 78.29 202.39) (end 79.56 201.12) (width 0.5) (layer "F.Cu") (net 13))
 (segment (start 79.56 198.58) (end 256.42 198.58) (width 0.5) (layer "F.Cu") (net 14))
 (segment (start 256.42 198.58) (end 257.69 199.85) (width 0.5) (layer "F.Cu") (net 14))
 (segment (start 78.29 199.85) (end 79.56 198.58) (width 0.5) (layer "F.Cu") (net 14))
 (segment (start 79.56 196.04) (end 256.42 196.04) (width 0.5) (layer "F.Cu") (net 15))
 (segment (start 78.29 197.31) (end 79.56 196.04) (width 0.5) (layer "F.Cu") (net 15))
 (segment (start 256.42 196.04) (end 257.69 197.31) (width 0.5) (layer "F.Cu") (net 15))
 (segment (start 256.42 193.5) (end 257.69 194.77) (width 0.5) (layer "F.Cu") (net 16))
 (segment (start 78.29 194.77) (end 79.56 193.5) (width 0.5) (layer "F.Cu") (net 16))
 (segment (start 79.56 193.5) (end 256.42 193.5) (width 0.5) (layer "F.Cu") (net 16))
 (segment (start 79.56 190.96) (end 256.42 190.96) (width 0.5) (layer "F.Cu") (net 17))
 (segment (start 256.42 190.96) (end 257.69 192.23) (width 0.5) (layer "F.Cu") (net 17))
 (segment (start 78.29 192.23) (end 79.56 190.96) (width 0.5) (layer "F.Cu") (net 17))
 (segment (start 256.41 188.41) (end 257.69 189.69) (width 0.5) (layer "F.Cu") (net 18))
 (segment (start 78.29 189.69) (end 79.57 188.41) (width 0.5) (layer "F.Cu") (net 18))
 (segment (start 79.57 188.41) (end 256.41 188.41) (width 0.5) (layer "F.Cu") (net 18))
 (segment (start 78.29 187.15) (end 79.57 185.87) (width 0.5) (layer "F.Cu") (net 19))
 (segment (start 79.57 185.87) (end 256.41 185.87) (width 0.5) (layer "F.Cu") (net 19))
 (segment (start 256.41 185.87) (end 257.69 187.15) (width 0.5) (layer "F.Cu") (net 19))
 (segment (start 256.41 183.33) (end 257.69 184.61) (width 0.5) (layer "F.Cu") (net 20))
 (segment (start 79.57 183.33) (end 256.41 183.33) (width 0.5) (layer "F.Cu") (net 20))
 (segment (start 78.29 184.61) (end 79.57 183.33) (width 0.5) (layer "F.Cu") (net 20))
 (segment (start 78.29 182.07) (end 79.56 180.8) (width 0.5) (layer "F.Cu") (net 21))
 (segment (start 79.56 180.8) (end 256.42 180.8) (width 0.5) (layer "F.Cu") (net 21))
 (segment (start 256.42 180.8) (end 257.69 182.07) (width 0.5) (layer "F.Cu") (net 21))
 (segment (start 256.42 178.26) (end 257.69 179.53) (width 0.5) (layer "F.Cu") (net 22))
 (segment (start 79.56 178.26) (end 256.42 178.26) (width 0.5) (layer "F.Cu") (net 22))
 (segment (start 78.29 179.53) (end 79.56 178.26) (width 0.5) (layer "F.Cu") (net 22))
 (segment (start 256.43 175.73) (end 257.69 176.99) (width 0.5) (layer "F.Cu") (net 23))
 (segment (start 78.29 176.99) (end 79.55 175.73) (width 0.5) (layer "F.Cu") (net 23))
 (segment (start 79.55 175.73) (end 256.43 175.73) (width 0.5) (layer "F.Cu") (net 23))
 (segment (start 78.29 174.45) (end 79.57 173.17) (width 0.5) (layer "F.Cu") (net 24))
 (segment (start 256.41 173.17) (end 257.69 174.45) (width 0.5) (layer "F.Cu") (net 24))
 (segment (start 79.57 173.17) (end 256.41 173.17) (width 0.5) (layer "F.Cu") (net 24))
 (segment (start 78.29 171.91) (end 79.56 170.64) (width 0.5) (layer "F.Cu") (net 25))
 (segment (start 256.42 170.64) (end 257.69 171.91) (width 0.5) (layer "F.Cu") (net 25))
 (segment (start 79.56 170.64) (end 256.42 170.64) (width 0.5) (layer "F.Cu") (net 25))
 (segment (start 79.56 168.1) (end 256.42 168.1) (width 0.5) (layer "F.Cu") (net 26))
 (segment (start 78.29 169.37) (end 79.56 168.1) (width 0.5) (layer "F.Cu") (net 26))
 (segment (start 256.42 168.1) (end 257.69 169.37) (width 0.5) (layer "F.Cu") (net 26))
 (segment (start 78.29 166.83) (end 79.56 165.56) (width 0.5) (layer "F.Cu") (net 27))
 (segment (start 256.42 165.56) (end 257.69 166.83) (width 0.5) (layer "F.Cu") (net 27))
 (segment (start 79.56 165.56) (end 256.42 165.56) (width 0.5) (layer "F.Cu") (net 27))
 (segment (start 256.42 163.02) (end 257.69 164.29) (width 0.5) (layer "F.Cu") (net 28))
 (segment (start 78.29 164.29) (end 79.56 163.02) (width 0.5) (layer "F.Cu") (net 28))
 (segment (start 79.56 163.02) (end 256.42 163.02) (width 0.5) (layer "F.Cu") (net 28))
 (segment (start 78.29 161.75) (end 79.56 160.48) (width 0.5) (layer "F.Cu") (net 29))
 (segment (start 79.56 160.48) (end 256.42 160.48) (width 0.5) (layer "F.Cu") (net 29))
 (segment (start 256.42 160.48) (end 257.69 161.75) (width 0.5) (layer "F.Cu") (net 29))
 (segment (start 256.42 157.94) (end 257.69 159.21) (width 0.5) (layer "F.Cu") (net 30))
 (segment (start 78.29 159.21) (end 79.56 157.94) (width 0.5) (layer "F.Cu") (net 30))
 (segment (start 79.56 157.94) (end 256.42 157.94) (width 0.5) (layer "F.Cu") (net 30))
 (segment (start 256.43 155.41) (end 257.69 156.67) (width 0.5) (layer "F.Cu") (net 31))
 (segment (start 79.55 155.41) (end 256.43 155.41) (width 0.5) (layer "F.Cu") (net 31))
 (segment (start 78.29 156.67) (end 79.55 155.41) (width 0.5) (layer "F.Cu") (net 31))
 (segment (start 79.52 152.9) (end 256.46 152.9) (width 0.5) (layer "F.Cu") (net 32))
 (segment (start 256.46 152.9) (end 257.69 154.13) (width 0.5) (layer "F.Cu") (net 32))
 (segment (start 78.29 154.13) (end 79.52 152.9) (width 0.5) (layer "F.Cu") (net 32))
 (segment (start 80.83 232.87) (end 255.15 232.87) (width 0.5) (layer "B.Cu") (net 33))
 (segment (start 255.15 230.33) (end 80.83 230.33) (width 0.5) (layer "B.Cu") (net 34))
 (segment (start 80.83 227.79) (end 255.15 227.79) (width 0.5) (layer "B.Cu") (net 35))
 (segment (start 255.15 225.25) (end 80.83 225.25) (width 0.5) (layer "B.Cu") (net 36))
 (segment (start 80.83 222.71) (end 255.15 222.71) (width 0.5) (layer "B.Cu") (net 37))
 (segment (start 255.15 220.17) (end 80.83 220.17) (width 0.5) (layer "B.Cu") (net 38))
 (segment (start 80.83 217.63) (end 255.15 217.63) (width 0.5) (layer "B.Cu") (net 39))
 (segment (start 80.83 215.09) (end 255.15 215.09) (width 0.5) (layer "B.Cu") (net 40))
 (segment (start 255.15 212.55) (end 80.83 212.55) (width 0.5) (layer "B.Cu") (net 41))
 (segment (start 80.83 210.01) (end 255.15 210.01) (width 0.5) (layer "B.Cu") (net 42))
 (segment (start 255.15 207.47) (end 80.83 207.47) (width 0.5) (layer "B.Cu") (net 43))
 (segment (start 80.83 204.93) (end 255.15 204.93) (width 0.5) (layer "B.Cu") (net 44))
 (segment (start 255.15 202.39) (end 80.83 202.39) (width 0.5) (layer "B.Cu") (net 45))
 (segment (start 80.83 199.85) (end 255.15 199.85) (width 0.5) (layer "B.Cu") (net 46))
 (segment (start 255.15 197.31) (end 80.83 197.31) (width 0.5) (layer "B.Cu") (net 47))
 (segment (start 80.83 194.77) (end 255.15 194.77) (width 0.5) (layer "B.Cu") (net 48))
 (segment (start 255.15 192.23) (end 80.83 192.23) (width 0.5) (layer "B.Cu") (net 49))
 (segment (start 80.83 189.69) (end 255.15 189.69) (width 0.5) (layer "B.Cu") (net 50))
 (segment (start 255.15 187.15) (end 80.83 187.15) (width 0.5) (layer "B.Cu") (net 51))
 (segment (start 80.83 184.61) (end 255.15 184.61) (width 0.5) (layer "B.Cu") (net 52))
 (segment (start 255.15 182.07) (end 80.83 182.07) (width 0.5) (layer "B.Cu") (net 53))
 (segment (start 80.83 179.53) (end 255.15 179.53) (width 0.5) (layer "B.Cu") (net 54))
 (segment (start 255.15 176.99) (end 80.83 176.99) (width 0.5) (layer "B.Cu") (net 55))
 (segment (start 80.83 174.45) (end 255.15 174.45) (width 0.5) (layer "B.Cu") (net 56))
 (segment (start 255.15 171.91) (end 80.83 171.91) (width 0.5) (layer "B.Cu") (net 57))
 (segment (start 80.83 169.37) (end 255.15 169.37) (width 0.5) (layer "B.Cu") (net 58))
 (segment (start 255.15 166.83) (end 80.83 166.83) (width 0.5) (layer "B.Cu") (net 59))
 (segment (start 80.83 164.29) (end 255.15 164.29) (width 0.5) (layer "B.Cu") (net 60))
 (segment (start 255.15 161.75) (end 80.83 161.75) (width 0.5) (layer "B.Cu") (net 61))
 (segment (start 80.83 159.21) (end 255.15 159.21) (width 0.5) (layer "B.Cu") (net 62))
 (segment (start 255.15 156.67) (end 80.83 156.67) (width 0.5) (layer "B.Cu") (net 63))
 (segment (start 80.83 154.13) (end 255.15 154.13) (width 0.5) (layer "B.Cu") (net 64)))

